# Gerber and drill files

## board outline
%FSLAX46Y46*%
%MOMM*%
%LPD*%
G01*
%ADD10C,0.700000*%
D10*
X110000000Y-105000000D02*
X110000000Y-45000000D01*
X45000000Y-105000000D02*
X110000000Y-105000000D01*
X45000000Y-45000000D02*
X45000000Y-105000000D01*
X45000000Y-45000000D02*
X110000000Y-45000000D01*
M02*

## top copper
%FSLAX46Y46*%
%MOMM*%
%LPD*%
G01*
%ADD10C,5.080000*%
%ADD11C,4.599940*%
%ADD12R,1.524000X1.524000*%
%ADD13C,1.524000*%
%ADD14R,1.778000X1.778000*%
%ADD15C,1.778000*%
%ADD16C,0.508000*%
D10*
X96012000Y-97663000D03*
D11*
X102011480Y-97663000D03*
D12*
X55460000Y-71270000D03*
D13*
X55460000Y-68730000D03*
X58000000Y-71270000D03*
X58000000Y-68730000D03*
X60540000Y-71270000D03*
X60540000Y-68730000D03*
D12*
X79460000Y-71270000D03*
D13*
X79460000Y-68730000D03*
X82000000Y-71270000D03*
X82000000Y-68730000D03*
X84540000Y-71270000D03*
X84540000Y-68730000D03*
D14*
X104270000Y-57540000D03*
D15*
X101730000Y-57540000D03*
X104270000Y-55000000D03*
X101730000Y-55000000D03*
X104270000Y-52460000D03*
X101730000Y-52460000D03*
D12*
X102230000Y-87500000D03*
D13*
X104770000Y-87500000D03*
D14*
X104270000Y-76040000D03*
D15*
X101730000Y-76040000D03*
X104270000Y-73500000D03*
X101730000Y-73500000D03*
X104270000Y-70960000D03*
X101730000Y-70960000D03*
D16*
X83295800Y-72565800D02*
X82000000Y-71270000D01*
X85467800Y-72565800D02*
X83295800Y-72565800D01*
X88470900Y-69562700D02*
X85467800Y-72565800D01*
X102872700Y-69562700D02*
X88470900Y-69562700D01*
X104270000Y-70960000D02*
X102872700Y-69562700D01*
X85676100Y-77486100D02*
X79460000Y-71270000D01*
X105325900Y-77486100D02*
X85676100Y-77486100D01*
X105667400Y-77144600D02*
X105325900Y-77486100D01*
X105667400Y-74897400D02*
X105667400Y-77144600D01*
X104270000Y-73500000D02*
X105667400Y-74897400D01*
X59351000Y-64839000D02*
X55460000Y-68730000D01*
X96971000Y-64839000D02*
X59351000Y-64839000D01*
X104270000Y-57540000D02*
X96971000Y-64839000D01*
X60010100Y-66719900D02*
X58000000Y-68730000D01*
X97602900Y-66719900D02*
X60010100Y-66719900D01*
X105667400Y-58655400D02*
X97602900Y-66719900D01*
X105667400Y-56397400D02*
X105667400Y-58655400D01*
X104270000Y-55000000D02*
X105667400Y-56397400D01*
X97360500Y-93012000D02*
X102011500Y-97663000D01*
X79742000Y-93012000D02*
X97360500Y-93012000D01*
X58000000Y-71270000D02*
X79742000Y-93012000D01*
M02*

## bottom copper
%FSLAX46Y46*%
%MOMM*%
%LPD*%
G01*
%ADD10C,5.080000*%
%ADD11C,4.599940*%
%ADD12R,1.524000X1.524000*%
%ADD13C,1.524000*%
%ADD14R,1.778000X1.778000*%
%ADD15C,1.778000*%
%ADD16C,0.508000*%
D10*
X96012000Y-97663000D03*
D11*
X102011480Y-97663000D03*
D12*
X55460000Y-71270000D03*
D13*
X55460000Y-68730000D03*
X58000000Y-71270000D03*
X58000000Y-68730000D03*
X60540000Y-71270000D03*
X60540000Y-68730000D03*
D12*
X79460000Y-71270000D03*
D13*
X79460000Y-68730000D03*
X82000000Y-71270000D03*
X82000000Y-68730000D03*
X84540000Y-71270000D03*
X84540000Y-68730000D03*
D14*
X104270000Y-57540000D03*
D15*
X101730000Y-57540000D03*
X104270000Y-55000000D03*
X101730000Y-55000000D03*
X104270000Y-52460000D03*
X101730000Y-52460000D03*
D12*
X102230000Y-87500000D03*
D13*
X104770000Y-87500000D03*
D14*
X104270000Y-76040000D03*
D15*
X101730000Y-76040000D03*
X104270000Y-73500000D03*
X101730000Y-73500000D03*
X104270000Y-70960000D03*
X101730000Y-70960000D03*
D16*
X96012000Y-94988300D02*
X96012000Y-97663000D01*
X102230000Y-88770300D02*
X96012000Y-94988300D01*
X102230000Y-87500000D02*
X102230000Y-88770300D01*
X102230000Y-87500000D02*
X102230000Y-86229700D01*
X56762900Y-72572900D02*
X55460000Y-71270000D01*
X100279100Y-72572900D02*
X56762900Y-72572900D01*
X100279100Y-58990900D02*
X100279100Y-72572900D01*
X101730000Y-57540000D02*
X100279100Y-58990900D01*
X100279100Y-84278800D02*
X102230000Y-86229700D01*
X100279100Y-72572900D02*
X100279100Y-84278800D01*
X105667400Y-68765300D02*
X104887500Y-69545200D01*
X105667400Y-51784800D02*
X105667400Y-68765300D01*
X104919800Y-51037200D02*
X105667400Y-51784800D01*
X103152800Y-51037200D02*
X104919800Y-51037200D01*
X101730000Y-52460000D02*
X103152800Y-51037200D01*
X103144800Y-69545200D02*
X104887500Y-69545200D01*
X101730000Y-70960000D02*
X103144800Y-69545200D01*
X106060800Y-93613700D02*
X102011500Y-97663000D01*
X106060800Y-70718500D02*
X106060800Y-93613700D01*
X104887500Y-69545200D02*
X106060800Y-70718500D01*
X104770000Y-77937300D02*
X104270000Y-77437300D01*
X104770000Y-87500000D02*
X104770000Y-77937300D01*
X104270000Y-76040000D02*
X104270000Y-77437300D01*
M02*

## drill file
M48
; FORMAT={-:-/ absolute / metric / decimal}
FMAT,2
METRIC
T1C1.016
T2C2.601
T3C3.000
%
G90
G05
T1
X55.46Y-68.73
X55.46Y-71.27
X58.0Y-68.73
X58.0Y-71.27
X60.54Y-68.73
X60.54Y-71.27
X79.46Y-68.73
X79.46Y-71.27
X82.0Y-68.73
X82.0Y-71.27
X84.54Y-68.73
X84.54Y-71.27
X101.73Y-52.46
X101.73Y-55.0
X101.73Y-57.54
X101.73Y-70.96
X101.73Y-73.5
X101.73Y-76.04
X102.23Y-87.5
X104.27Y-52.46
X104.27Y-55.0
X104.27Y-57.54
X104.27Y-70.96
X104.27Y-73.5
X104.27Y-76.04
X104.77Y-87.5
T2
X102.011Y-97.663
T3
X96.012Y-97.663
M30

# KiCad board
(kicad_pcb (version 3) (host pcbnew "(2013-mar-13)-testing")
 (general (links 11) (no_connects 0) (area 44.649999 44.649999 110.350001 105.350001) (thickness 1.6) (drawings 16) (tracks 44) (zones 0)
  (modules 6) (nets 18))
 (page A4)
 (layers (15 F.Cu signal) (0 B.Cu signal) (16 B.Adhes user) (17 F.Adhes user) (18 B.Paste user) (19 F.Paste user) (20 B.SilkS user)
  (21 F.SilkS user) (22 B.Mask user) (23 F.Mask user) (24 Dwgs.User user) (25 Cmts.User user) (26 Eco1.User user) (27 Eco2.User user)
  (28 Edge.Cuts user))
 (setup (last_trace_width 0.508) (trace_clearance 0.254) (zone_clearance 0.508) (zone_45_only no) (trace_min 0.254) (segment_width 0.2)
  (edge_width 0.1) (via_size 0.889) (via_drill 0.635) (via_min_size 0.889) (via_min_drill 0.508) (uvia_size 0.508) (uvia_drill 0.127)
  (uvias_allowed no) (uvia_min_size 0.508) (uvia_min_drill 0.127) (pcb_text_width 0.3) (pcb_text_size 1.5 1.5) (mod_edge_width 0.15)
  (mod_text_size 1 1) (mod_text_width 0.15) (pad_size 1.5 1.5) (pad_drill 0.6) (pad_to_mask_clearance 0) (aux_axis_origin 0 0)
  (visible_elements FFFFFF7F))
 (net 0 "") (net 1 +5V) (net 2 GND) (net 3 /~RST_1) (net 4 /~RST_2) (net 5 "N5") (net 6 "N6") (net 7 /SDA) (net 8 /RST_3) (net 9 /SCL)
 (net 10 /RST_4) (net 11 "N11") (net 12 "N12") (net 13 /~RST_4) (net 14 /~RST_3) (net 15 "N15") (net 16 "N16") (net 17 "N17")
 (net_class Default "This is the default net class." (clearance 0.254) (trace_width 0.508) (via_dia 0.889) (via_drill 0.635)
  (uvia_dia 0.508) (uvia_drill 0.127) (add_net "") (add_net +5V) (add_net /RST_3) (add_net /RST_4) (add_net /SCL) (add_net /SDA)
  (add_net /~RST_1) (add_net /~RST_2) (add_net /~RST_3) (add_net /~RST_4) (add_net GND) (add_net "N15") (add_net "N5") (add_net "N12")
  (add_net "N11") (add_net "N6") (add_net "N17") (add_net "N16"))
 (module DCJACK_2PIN (layer F.Cu) (at 96.012 97.663)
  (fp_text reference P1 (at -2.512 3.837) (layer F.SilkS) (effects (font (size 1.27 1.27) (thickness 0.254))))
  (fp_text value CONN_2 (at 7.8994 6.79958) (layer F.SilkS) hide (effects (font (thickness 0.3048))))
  (pad 1 thru_hole circle (at 0 0) (size 5.08 5.08) (drill 2.99974) (layers *.Cu *.Mask F.SilkS) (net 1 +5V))
  (pad 2 thru_hole circle (at 5.99948 0) (size 4.59994 4.59994) (drill 2.60096) (layers *.Cu *.Mask F.SilkS) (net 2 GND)))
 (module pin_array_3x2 (layer F.Cu) (at 58 70)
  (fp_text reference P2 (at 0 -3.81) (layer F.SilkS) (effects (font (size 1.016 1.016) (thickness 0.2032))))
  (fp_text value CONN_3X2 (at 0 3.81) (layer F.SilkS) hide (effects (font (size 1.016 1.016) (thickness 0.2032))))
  (pad 1 thru_hole rect (at -2.54 1.27) (size 1.524 1.524) (drill 1.016) (layers *.Cu *.Mask F.SilkS) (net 1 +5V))
  (pad 2 thru_hole circle (at -2.54 -1.27) (size 1.524 1.524) (drill 1.016) (layers *.Cu *.Mask F.SilkS) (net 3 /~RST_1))
  (pad 3 thru_hole circle (at 0 1.27) (size 1.524 1.524) (drill 1.016) (layers *.Cu *.Mask F.SilkS) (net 2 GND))
  (pad 4 thru_hole circle (at 0 -1.27) (size 1.524 1.524) (drill 1.016) (layers *.Cu *.Mask F.SilkS) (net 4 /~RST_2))
  (pad 5 thru_hole circle (at 2.54 1.27) (size 1.524 1.524) (drill 1.016) (layers *.Cu *.Mask F.SilkS) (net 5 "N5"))
  (pad 6 thru_hole circle (at 2.54 -1.27) (size 1.524 1.524) (drill 1.016) (layers *.Cu *.Mask F.SilkS) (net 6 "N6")))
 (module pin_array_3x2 (layer F.Cu) (at 82 70)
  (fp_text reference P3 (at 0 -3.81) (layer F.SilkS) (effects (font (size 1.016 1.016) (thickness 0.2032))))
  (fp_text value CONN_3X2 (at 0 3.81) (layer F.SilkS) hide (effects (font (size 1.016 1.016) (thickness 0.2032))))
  (pad 1 thru_hole rect (at -2.54 1.27) (size 1.524 1.524) (drill 1.016) (layers *.Cu *.Mask F.SilkS) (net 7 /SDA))
  (pad 2 thru_hole circle (at -2.54 -1.27) (size 1.524 1.524) (drill 1.016) (layers *.Cu *.Mask F.SilkS) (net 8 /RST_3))
  (pad 3 thru_hole circle (at 0 1.27) (size 1.524 1.524) (drill 1.016) (layers *.Cu *.Mask F.SilkS) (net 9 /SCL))
  (pad 4 thru_hole circle (at 0 -1.27) (size 1.524 1.524) (drill 1.016) (layers *.Cu *.Mask F.SilkS) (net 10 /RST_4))
  (pad 5 thru_hole circle (at 2.54 1.27) (size 1.524 1.524) (drill 1.016) (layers *.Cu *.Mask F.SilkS) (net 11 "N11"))
  (pad 6 thru_hole circle (at 2.54 -1.27) (size 1.524 1.524) (drill 1.016) (layers *.Cu *.Mask F.SilkS) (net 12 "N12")))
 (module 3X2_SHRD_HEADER (layer F.Cu) (at 103 55 90)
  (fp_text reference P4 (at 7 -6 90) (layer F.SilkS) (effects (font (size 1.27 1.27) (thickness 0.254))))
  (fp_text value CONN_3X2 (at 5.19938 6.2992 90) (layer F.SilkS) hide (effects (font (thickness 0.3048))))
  (pad 1 thru_hole rect (at -2.54 1.27 90) (size 1.778 1.778) (drill 1.016) (layers *.Cu *.Mask F.SilkS) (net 3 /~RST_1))
  (pad 2 thru_hole circle (at -2.54 -1.27 90) (size 1.778 1.778) (drill 1.016) (layers *.Cu *.Mask F.SilkS) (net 1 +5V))
  (pad 3 thru_hole circle (at 0 1.27 90) (size 1.778 1.778) (drill 1.016) (layers *.Cu *.Mask F.SilkS) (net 4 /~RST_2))
  (pad 4 thru_hole circle (at 0 -1.27 90) (size 1.778 1.778) (drill 1.016) (layers *.Cu *.Mask F.SilkS) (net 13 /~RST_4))
  (pad 5 thru_hole circle (at 2.54 1.27 90) (size 1.778 1.778) (drill 1.016) (layers *.Cu *.Mask F.SilkS) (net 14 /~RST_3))
  (pad 6 thru_hole circle (at 2.54 -1.27 90) (size 1.778 1.778) (drill 1.016) (layers *.Cu *.Mask F.SilkS) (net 2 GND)))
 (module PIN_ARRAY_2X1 (layer F.Cu) (at 103.5 87.5)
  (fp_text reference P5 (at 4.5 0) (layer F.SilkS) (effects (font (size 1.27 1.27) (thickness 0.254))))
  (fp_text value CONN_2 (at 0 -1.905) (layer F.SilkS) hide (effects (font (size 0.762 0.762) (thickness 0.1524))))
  (pad 1 thru_hole rect (at -1.27 0) (size 1.524 1.524) (drill 1.016) (layers *.Cu *.Mask F.SilkS) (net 1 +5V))
  (pad 2 thru_hole circle (at 1.27 0) (size 1.524 1.524) (drill 1.016) (layers *.Cu *.Mask F.SilkS) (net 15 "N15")))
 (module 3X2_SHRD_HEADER (layer F.Cu) (at 103 73.5 90)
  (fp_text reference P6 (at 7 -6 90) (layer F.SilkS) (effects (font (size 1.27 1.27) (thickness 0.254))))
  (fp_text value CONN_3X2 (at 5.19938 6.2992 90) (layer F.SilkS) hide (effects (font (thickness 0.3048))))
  (pad 1 thru_hole rect (at -2.54 1.27 90) (size 1.778 1.778) (drill 1.016) (layers *.Cu *.Mask F.SilkS) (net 15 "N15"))
  (pad 2 thru_hole circle (at -2.54 -1.27 90) (size 1.778 1.778) (drill 1.016) (layers *.Cu *.Mask F.SilkS) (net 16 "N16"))
  (pad 3 thru_hole circle (at 0 1.27 90) (size 1.778 1.778) (drill 1.016) (layers *.Cu *.Mask F.SilkS) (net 7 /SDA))
  (pad 4 thru_hole circle (at 0 -1.27 90) (size 1.778 1.778) (drill 1.016) (layers *.Cu *.Mask F.SilkS) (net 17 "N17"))
  (pad 5 thru_hole circle (at 2.54 1.27 90) (size 1.778 1.778) (drill 1.016) (layers *.Cu *.Mask F.SilkS) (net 9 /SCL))
  (pad 6 thru_hole circle (at 2.54 -1.27 90) (size 1.778 1.778) (drill 1.016) (layers *.Cu *.Mask F.SilkS) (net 2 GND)))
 (gr_line (start 110 105) (end 110 45) (angle 90) (layer Edge.Cuts) (width 0.7))
 (gr_line (start 45 105) (end 110 105) (angle 90) (layer Edge.Cuts) (width 0.7))
 (gr_line (start 45 45) (end 45 105) (angle 90) (layer Edge.Cuts) (width 0.7))
 (gr_line (start 45 45) (end 110 45) (angle 90) (layer Edge.Cuts) (width 0.7))
 (segment (start 96.012 94.9883) (end 96.012 97.663) (width 0.508) (layer B.Cu) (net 1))
 (segment (start 102.23 88.7703) (end 96.012 94.9883) (width 0.508) (layer B.Cu) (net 1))
 (segment (start 102.23 87.5) (end 102.23 88.7703) (width 0.508) (layer B.Cu) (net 1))
 (segment (start 102.23 87.5) (end 102.23 86.2297) (width 0.508) (layer B.Cu) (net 1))
 (segment (start 56.7629 72.5729) (end 55.46 71.27) (width 0.508) (layer B.Cu) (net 1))
 (segment (start 100.2791 72.5729) (end 56.7629 72.5729) (width 0.508) (layer B.Cu) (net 1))
 (segment (start 100.2791 58.9909) (end 100.2791 72.5729) (width 0.508) (layer B.Cu) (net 1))
 (segment (start 101.73 57.54) (end 100.2791 58.9909) (width 0.508) (layer B.Cu) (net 1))
 (segment (start 100.2791 84.2788) (end 102.23 86.2297) (width 0.508) (layer B.Cu) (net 1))
 (segment (start 100.2791 72.5729) (end 100.2791 84.2788) (width 0.508) (layer B.Cu) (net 1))
 (segment (start 83.2958 72.5658) (end 82 71.27) (width 0.508) (layer F.Cu) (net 9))
 (segment (start 85.4678 72.5658) (end 83.2958 72.5658) (width 0.508) (layer F.Cu) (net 9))
 (segment (start 88.4709 69.5627) (end 85.4678 72.5658) (width 0.508) (layer F.Cu) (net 9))
 (segment (start 102.8727 69.5627) (end 88.4709 69.5627) (width 0.508) (layer F.Cu) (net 9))
 (segment (start 104.27 70.96) (end 102.8727 69.5627) (width 0.508) (layer F.Cu) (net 9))
 (segment (start 85.6761 77.4861) (end 79.46 71.27) (width 0.508) (layer F.Cu) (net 7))
 (segment (start 105.3259 77.4861) (end 85.6761 77.4861) (width 0.508) (layer F.Cu) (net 7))
 (segment (start 105.6674 77.1446) (end 105.3259 77.4861) (width 0.508) (layer F.Cu) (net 7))
 (segment (start 105.6674 74.8974) (end 105.6674 77.1446) (width 0.508) (layer F.Cu) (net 7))
 (segment (start 104.27 73.5) (end 105.6674 74.8974) (width 0.508) (layer F.Cu) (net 7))
 (segment (start 59.351 64.839) (end 55.46 68.73) (width 0.508) (layer F.Cu) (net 3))
 (segment (start 96.971 64.839) (end 59.351 64.839) (width 0.508) (layer F.Cu) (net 3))
 (segment (start 104.27 57.54) (end 96.971 64.839) (width 0.508) (layer F.Cu) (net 3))
 (segment (start 60.0101 66.7199) (end 58 68.73) (width 0.508) (layer F.Cu) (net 4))
 (segment (start 97.6029 66.7199) (end 60.0101 66.7199) (width 0.508) (layer F.Cu) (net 4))
 (segment (start 105.6674 58.6554) (end 97.6029 66.7199) (width 0.508) (layer F.Cu) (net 4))
 (segment (start 105.6674 56.3974) (end 105.6674 58.6554) (width 0.508) (layer F.Cu) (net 4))
 (segment (start 104.27 55) (end 105.6674 56.3974) (width 0.508) (layer F.Cu) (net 4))
 (segment (start 97.3605 93.012) (end 102.0115 97.663) (width 0.508) (layer F.Cu) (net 2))
 (segment (start 79.742 93.012) (end 97.3605 93.012) (width 0.508) (layer F.Cu) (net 2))
 (segment (start 58 71.27) (end 79.742 93.012) (width 0.508) (layer F.Cu) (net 2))
 (segment (start 105.6674 68.7653) (end 104.8875 69.5452) (width 0.508) (layer B.Cu) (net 2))
 (segment (start 105.6674 51.7848) (end 105.6674 68.7653) (width 0.508) (layer B.Cu) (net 2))
 (segment (start 104.9198 51.0372) (end 105.6674 51.7848) (width 0.508) (layer B.Cu) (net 2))
 (segment (start 103.1528 51.0372) (end 104.9198 51.0372) (width 0.508) (layer B.Cu) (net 2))
 (segment (start 101.73 52.46) (end 103.1528 51.0372) (width 0.508) (layer B.Cu) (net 2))
 (segment (start 103.1448 69.5452) (end 104.8875 69.5452) (width 0.508) (layer B.Cu) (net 2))
 (segment (start 101.73 70.96) (end 103.1448 69.5452) (width 0.508) (layer B.Cu) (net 2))
 (segment (start 106.0608 93.6137) (end 102.0115 97.663) (width 0.508) (layer B.Cu) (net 2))
 (segment (start 106.0608 70.7185) (end 106.0608 93.6137) (width 0.508) (layer B.Cu) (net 2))
 (segment (start 104.8875 69.5452) (end 106.0608 70.7185) (width 0.508) (layer B.Cu) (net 2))
 (segment (start 104.77 77.9373) (end 104.27 77.4373) (width 0.508) (layer B.Cu) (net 15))
 (segment (start 104.77 87.5) (end 104.77 77.9373) (width 0.508) (layer B.Cu) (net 15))
 (segment (start 104.27 76.04) (end 104.27 77.4373) (width 0.508) (layer B.Cu) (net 15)))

